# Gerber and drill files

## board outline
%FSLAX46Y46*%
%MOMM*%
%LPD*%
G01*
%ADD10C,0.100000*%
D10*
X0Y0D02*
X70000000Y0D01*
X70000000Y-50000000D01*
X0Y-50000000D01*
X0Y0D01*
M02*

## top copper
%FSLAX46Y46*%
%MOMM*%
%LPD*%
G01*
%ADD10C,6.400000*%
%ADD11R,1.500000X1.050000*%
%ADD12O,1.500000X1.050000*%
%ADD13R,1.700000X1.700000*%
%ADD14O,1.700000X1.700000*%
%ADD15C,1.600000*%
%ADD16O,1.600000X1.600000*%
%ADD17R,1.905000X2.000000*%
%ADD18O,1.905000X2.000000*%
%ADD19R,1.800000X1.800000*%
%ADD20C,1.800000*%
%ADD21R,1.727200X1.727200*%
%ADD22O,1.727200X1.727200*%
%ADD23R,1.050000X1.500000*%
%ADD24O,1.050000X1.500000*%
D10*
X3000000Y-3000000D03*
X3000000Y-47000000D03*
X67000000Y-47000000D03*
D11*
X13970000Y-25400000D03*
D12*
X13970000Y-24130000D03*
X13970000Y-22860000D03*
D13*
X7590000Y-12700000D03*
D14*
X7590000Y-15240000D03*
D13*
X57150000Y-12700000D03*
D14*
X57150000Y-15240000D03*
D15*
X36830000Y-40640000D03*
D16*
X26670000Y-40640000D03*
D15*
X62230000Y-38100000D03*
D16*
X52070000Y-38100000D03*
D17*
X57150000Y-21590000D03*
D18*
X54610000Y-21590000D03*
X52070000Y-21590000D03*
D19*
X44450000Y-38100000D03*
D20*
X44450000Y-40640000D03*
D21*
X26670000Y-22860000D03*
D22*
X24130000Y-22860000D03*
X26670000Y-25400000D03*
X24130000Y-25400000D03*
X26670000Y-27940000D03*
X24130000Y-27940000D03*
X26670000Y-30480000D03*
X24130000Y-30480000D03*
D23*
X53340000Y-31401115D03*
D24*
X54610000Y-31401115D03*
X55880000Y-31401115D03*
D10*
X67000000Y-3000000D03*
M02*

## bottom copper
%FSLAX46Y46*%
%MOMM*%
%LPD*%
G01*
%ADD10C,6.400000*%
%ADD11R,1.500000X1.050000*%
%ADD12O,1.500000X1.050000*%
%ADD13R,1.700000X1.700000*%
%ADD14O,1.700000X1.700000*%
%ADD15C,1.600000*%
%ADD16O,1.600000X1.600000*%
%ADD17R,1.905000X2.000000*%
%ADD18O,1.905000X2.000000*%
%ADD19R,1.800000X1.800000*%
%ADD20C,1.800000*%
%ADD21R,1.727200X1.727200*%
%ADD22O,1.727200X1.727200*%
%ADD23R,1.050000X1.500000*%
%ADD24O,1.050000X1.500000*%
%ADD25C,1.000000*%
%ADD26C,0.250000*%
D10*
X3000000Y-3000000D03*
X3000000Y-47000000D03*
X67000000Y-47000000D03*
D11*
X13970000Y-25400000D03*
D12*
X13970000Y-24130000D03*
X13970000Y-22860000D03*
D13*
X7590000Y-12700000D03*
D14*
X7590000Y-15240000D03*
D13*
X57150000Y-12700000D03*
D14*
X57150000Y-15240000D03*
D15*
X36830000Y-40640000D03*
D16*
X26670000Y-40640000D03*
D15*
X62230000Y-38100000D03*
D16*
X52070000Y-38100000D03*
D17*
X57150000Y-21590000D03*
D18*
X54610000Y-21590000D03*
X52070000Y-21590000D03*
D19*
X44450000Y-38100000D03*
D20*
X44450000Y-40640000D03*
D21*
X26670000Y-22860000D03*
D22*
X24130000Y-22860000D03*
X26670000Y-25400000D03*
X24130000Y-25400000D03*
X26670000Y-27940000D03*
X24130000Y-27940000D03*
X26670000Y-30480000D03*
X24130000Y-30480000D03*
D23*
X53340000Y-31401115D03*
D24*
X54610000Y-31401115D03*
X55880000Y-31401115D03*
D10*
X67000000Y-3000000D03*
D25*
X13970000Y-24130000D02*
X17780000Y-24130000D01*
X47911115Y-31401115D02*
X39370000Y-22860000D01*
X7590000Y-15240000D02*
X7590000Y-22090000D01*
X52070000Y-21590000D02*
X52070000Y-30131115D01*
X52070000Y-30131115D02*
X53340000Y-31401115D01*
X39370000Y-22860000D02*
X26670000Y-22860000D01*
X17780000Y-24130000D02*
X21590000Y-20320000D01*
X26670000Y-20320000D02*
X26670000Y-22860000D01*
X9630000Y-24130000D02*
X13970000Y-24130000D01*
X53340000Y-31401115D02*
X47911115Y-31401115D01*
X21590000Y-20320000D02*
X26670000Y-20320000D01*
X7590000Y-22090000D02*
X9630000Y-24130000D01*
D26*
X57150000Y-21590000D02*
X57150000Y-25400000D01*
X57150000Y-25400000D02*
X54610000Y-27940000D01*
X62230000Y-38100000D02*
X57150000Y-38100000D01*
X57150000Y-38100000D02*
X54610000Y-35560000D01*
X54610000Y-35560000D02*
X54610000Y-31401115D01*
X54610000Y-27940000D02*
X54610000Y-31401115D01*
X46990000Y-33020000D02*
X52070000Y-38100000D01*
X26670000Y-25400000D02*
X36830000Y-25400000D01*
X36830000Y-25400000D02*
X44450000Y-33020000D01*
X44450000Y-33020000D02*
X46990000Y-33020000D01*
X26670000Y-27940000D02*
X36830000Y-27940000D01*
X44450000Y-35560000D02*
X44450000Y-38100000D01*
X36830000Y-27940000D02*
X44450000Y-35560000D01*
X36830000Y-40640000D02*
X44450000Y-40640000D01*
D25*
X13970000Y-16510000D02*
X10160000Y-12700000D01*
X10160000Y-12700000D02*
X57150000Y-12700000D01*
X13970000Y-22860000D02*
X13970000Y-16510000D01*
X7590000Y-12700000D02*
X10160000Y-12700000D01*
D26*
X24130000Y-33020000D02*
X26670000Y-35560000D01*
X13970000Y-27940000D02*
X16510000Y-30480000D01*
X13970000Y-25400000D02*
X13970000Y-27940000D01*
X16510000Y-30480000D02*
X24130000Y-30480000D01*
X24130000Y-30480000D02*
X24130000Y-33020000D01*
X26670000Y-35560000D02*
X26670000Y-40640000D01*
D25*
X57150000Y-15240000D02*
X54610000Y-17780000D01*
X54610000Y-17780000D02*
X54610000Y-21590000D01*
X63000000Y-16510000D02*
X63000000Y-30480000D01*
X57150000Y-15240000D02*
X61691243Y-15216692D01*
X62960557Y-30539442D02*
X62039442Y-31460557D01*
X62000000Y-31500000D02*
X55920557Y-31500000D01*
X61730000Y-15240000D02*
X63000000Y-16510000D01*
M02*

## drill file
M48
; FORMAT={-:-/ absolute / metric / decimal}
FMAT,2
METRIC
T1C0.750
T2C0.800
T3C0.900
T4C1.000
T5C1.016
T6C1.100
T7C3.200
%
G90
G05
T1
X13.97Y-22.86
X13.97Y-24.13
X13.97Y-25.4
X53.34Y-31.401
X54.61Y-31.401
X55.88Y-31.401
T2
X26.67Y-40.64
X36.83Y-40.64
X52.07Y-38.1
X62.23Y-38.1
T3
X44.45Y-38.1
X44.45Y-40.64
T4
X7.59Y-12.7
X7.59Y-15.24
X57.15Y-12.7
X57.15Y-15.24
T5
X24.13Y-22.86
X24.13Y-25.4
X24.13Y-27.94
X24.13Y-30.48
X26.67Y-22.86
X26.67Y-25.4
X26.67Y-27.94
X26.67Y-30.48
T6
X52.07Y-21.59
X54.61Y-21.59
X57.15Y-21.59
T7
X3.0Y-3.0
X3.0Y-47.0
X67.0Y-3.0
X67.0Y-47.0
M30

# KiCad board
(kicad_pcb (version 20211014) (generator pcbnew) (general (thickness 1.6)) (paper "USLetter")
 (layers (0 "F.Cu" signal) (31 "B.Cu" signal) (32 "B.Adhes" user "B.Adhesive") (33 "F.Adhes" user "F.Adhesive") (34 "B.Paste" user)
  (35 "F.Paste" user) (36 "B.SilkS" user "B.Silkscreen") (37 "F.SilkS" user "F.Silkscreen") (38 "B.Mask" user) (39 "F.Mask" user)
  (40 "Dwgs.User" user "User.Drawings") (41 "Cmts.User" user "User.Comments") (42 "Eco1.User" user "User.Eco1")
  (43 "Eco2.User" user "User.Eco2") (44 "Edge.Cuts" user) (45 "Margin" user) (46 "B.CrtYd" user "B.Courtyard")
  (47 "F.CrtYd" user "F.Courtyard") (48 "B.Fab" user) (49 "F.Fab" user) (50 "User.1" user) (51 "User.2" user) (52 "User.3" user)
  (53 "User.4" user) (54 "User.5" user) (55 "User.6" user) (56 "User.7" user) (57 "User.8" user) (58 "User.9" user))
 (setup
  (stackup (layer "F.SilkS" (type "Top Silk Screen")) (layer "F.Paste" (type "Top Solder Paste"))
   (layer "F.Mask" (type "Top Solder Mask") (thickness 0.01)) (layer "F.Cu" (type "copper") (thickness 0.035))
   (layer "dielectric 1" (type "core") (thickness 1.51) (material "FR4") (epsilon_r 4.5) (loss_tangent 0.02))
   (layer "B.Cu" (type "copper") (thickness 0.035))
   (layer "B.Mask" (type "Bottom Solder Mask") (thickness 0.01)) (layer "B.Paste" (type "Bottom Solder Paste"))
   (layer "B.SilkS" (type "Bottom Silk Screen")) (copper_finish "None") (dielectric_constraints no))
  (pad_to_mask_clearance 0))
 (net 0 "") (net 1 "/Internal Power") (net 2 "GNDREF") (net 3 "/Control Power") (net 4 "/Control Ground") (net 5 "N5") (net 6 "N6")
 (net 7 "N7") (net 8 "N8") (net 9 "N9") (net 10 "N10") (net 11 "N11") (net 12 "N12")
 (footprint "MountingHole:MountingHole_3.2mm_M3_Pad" (layer "F.Cu") (at 3 3)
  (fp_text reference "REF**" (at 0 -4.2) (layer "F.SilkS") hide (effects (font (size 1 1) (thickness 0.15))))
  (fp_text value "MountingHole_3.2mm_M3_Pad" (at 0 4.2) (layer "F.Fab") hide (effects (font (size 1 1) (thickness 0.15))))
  (pad "1" thru_hole circle (at 0 0) (size 6.4 6.4) (drill 3.2) (layers *.Cu *.Mask)))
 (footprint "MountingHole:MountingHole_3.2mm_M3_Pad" (layer "F.Cu") (at 3 47)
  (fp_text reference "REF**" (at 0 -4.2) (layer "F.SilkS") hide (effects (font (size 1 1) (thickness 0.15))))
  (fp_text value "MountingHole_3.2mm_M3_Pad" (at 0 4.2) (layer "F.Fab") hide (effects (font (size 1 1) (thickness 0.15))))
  (pad "1" thru_hole circle (at 0 0) (size 6.4 6.4) (drill 3.2) (layers *.Cu *.Mask)))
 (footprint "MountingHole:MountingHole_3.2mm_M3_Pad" (layer "F.Cu") (at 67 47)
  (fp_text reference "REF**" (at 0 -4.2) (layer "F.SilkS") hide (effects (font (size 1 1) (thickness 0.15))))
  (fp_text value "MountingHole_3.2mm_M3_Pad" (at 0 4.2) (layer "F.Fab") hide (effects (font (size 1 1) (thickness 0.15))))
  (pad "1" thru_hole circle (at 0 0) (size 6.4 6.4) (drill 3.2) (layers *.Cu *.Mask)))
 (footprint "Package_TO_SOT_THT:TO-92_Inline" (layer "F.Cu") (at 13.97 25.4 90)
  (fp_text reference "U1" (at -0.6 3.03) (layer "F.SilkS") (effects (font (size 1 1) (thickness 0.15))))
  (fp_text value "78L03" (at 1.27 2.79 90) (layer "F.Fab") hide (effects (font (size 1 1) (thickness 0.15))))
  (pad "1" thru_hole rect (at 0 0 90) (size 1.05 1.5) (drill 0.75) (layers *.Cu *.Mask) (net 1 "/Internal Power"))
  (pad "2" thru_hole oval (at 1.27 0 90) (size 1.05 1.5) (drill 0.75) (layers *.Cu *.Mask) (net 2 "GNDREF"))
  (pad "3" thru_hole oval (at 2.54 0 90) (size 1.05 1.5) (drill 0.75) (layers *.Cu *.Mask) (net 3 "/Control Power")))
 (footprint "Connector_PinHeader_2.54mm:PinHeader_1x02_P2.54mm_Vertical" (layer "F.Cu") (at 7.59 12.7)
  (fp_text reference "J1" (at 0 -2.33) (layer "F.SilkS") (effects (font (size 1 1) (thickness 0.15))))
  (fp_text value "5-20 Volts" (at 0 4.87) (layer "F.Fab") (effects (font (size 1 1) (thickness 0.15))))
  (pad "1" thru_hole rect (at 0 0) (size 1.7 1.7) (drill 1) (layers *.Cu *.Mask) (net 3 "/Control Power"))
  (pad "2" thru_hole oval (at 0 2.54) (size 1.7 1.7) (drill 1) (layers *.Cu *.Mask) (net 2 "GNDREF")))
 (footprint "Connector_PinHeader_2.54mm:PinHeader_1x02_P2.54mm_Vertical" (layer "F.Cu") (at 57.15 12.7)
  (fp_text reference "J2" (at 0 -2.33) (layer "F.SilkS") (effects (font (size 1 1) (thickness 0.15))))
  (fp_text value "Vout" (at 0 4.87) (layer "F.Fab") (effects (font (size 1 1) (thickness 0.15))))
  (pad "1" thru_hole rect (at 0 0) (size 1.7 1.7) (drill 1) (layers *.Cu *.Mask) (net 3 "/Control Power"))
  (pad "2" thru_hole oval (at 0 2.54) (size 1.7 1.7) (drill 1) (layers *.Cu *.Mask) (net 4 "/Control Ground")))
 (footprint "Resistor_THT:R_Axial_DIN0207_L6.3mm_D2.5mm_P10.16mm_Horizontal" (layer "F.Cu") (at 36.83 40.64 180)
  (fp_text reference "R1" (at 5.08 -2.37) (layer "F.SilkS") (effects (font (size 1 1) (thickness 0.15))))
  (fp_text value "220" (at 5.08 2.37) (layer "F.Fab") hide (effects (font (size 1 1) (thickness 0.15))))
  (pad "1" thru_hole circle (at 0 0 180) (size 1.6 1.6) (drill 0.8) (layers *.Cu *.Mask) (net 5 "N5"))
  (pad "2" thru_hole oval (at 10.16 0 180) (size 1.6 1.6) (drill 0.8) (layers *.Cu *.Mask) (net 1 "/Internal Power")))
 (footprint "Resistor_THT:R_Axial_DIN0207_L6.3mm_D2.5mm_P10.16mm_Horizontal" (layer "F.Cu") (at 62.23 38.1 180)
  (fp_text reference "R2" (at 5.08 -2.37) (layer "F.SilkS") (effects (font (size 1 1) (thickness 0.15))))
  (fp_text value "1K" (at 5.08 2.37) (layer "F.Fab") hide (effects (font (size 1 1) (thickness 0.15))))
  (pad "1" thru_hole circle (at 0 0 180) (size 1.6 1.6) (drill 0.8) (layers *.Cu *.Mask) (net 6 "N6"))
  (pad "2" thru_hole oval (at 10.16 0 180) (size 1.6 1.6) (drill 0.8) (layers *.Cu *.Mask) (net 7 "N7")))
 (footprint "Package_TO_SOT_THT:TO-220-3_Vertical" (layer "F.Cu") (at 57.15 21.59 180)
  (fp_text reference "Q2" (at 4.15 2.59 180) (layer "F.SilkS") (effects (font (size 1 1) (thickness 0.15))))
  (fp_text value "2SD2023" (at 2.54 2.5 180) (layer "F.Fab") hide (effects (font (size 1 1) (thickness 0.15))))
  (pad "1" thru_hole rect (at 0 0 180) (size 1.905 2) (drill 1.1) (layers *.Cu *.Mask) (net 6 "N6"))
  (pad "2" thru_hole oval (at 2.54 0 180) (size 1.905 2) (drill 1.1) (layers *.Cu *.Mask) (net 4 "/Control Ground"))
  (pad "3" thru_hole oval (at 5.08 0 180) (size 1.905 2) (drill 1.1) (layers *.Cu *.Mask) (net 2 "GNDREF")))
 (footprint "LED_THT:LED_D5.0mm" (layer "F.Cu") (at 44.45 38.1 -90)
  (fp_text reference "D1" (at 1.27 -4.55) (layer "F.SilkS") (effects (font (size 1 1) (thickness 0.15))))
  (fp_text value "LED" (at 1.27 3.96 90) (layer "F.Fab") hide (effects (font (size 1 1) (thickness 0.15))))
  (pad "1" thru_hole rect (at 0 0 270) (size 1.8 1.8) (drill 0.9) (layers *.Cu *.Mask) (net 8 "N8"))
  (pad "2" thru_hole circle (at 2.54 0 270) (size 1.8 1.8) (drill 0.9) (layers *.Cu *.Mask) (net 5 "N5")))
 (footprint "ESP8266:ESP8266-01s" (layer "F.Cu") (at 24.13 22.86)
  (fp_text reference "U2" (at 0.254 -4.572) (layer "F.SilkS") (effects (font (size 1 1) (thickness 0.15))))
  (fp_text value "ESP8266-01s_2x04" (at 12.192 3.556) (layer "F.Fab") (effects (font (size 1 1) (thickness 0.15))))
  (pad "1" thru_hole rect (at 2.54 0) (size 1.7272 1.7272) (drill 1.016) (layers *.Cu *.Mask) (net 2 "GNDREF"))
  (pad "2" thru_hole oval (at 0 0) (size 1.7272 1.7272) (drill 1.016) (layers *.Cu *.Mask) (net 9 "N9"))
  (pad "3" thru_hole oval (at 2.54 2.54) (size 1.7272 1.7272) (drill 1.016) (layers *.Cu *.Mask) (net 7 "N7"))
  (pad "4" thru_hole oval (at 0 2.54) (size 1.7272 1.7272) (drill 1.016) (layers *.Cu *.Mask) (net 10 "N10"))
  (pad "5" thru_hole oval (at 2.54 5.08) (size 1.7272 1.7272) (drill 1.016) (layers *.Cu *.Mask) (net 8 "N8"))
  (pad "6" thru_hole oval (at 0 5.08) (size 1.7272 1.7272) (drill 1.016) (layers *.Cu *.Mask) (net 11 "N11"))
  (pad "7" thru_hole oval (at 2.54 7.62) (size 1.7272 1.7272) (drill 1.016) (layers *.Cu *.Mask) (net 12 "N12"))
  (pad "8" thru_hole oval (at 0 7.62) (size 1.7272 1.7272) (drill 1.016) (layers *.Cu *.Mask) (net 1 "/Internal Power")))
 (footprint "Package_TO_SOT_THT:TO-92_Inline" (layer "F.Cu") (at 53.34 31.401115)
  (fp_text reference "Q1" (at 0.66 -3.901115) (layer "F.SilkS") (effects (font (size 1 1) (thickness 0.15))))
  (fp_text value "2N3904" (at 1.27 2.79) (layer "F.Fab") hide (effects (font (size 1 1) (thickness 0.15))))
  (pad "1" thru_hole rect (at 0 0) (size 1.05 1.5) (drill 0.75) (layers *.Cu *.Mask) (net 2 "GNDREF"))
  (pad "2" thru_hole oval (at 1.27 0) (size 1.05 1.5) (drill 0.75) (layers *.Cu *.Mask) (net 6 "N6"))
  (pad "3" thru_hole oval (at 2.54 0) (size 1.05 1.5) (drill 0.75) (layers *.Cu *.Mask) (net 4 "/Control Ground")))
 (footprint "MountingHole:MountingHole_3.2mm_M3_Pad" (layer "F.Cu") (at 67 3)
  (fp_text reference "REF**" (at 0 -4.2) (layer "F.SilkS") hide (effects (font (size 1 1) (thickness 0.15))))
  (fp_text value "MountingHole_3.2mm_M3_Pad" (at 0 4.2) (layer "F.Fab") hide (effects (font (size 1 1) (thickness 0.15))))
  (pad "1" thru_hole circle (at 0 0) (size 6.4 6.4) (drill 3.2) (layers *.Cu *.Mask)))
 (gr_rect (start 0 0) (end 70 50) (layer "Edge.Cuts") (width 0.1) (fill none))
 (segment (start 13.97 24.13) (end 17.78 24.13) (width 1) (layer "B.Cu") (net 2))
 (segment (start 47.911115 31.401115) (end 39.37 22.86) (width 1) (layer "B.Cu") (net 2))
 (segment (start 7.59 15.24) (end 7.59 22.09) (width 1) (layer "B.Cu") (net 2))
 (segment (start 52.07 21.59) (end 52.07 30.131115) (width 1) (layer "B.Cu") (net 2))
 (segment (start 52.07 30.131115) (end 53.34 31.401115) (width 1) (layer "B.Cu") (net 2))
 (segment (start 39.37 22.86) (end 26.67 22.86) (width 1) (layer "B.Cu") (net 2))
 (segment (start 17.78 24.13) (end 21.59 20.32) (width 1) (layer "B.Cu") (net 2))
 (segment (start 26.67 20.32) (end 26.67 22.86) (width 1) (layer "B.Cu") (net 2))
 (segment (start 9.63 24.13) (end 13.97 24.13) (width 1) (layer "B.Cu") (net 2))
 (segment (start 53.34 31.401115) (end 47.911115 31.401115) (width 1) (layer "B.Cu") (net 2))
 (segment (start 21.59 20.32) (end 26.67 20.32) (width 1) (layer "B.Cu") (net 2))
 (segment (start 7.59 22.09) (end 9.63 24.13) (width 1) (layer "B.Cu") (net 2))
 (segment (start 57.15 21.59) (end 57.15 25.4) (width 0.25) (layer "B.Cu") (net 6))
 (segment (start 57.15 25.4) (end 54.61 27.94) (width 0.25) (layer "B.Cu") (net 6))
 (segment (start 62.23 38.1) (end 57.15 38.1) (width 0.25) (layer "B.Cu") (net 6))
 (segment (start 57.15 38.1) (end 54.61 35.56) (width 0.25) (layer "B.Cu") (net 6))
 (segment (start 54.61 35.56) (end 54.61 31.401115) (width 0.25) (layer "B.Cu") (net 6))
 (segment (start 54.61 27.94) (end 54.61 31.401115) (width 0.25) (layer "B.Cu") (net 6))
 (segment (start 46.99 33.02) (end 52.07 38.1) (width 0.25) (layer "B.Cu") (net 7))
 (segment (start 26.67 25.4) (end 36.83 25.4) (width 0.25) (layer "B.Cu") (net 7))
 (segment (start 36.83 25.4) (end 44.45 33.02) (width 0.25) (layer "B.Cu") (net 7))
 (segment (start 44.45 33.02) (end 46.99 33.02) (width 0.25) (layer "B.Cu") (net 7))
 (segment (start 26.67 27.94) (end 36.83 27.94) (width 0.25) (layer "B.Cu") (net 8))
 (segment (start 44.45 35.56) (end 44.45 38.1) (width 0.25) (layer "B.Cu") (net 8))
 (segment (start 36.83 27.94) (end 44.45 35.56) (width 0.25) (layer "B.Cu") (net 8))
 (segment (start 36.83 40.64) (end 44.45 40.64) (width 0.25) (layer "B.Cu") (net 5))
 (segment (start 13.97 16.51) (end 10.16 12.7) (width 1) (layer "B.Cu") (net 3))
 (segment (start 10.16 12.7) (end 57.15 12.7) (width 1) (layer "B.Cu") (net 3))
 (segment (start 13.97 22.86) (end 13.97 16.51) (width 1) (layer "B.Cu") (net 3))
 (segment (start 7.59 12.7) (end 10.16 12.7) (width 1) (layer "B.Cu") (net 3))
 (segment (start 24.13 33.02) (end 26.67 35.56) (width 0.25) (layer "B.Cu") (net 1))
 (segment (start 13.97 27.94) (end 16.51 30.48) (width 0.25) (layer "B.Cu") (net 1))
 (segment (start 13.97 25.4) (end 13.97 27.94) (width 0.25) (layer "B.Cu") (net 1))
 (segment (start 16.51 30.48) (end 24.13 30.48) (width 0.25) (layer "B.Cu") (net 1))
 (segment (start 24.13 30.48) (end 24.13 33.02) (width 0.25) (layer "B.Cu") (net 1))
 (segment (start 26.67 35.56) (end 26.67 40.64) (width 0.25) (layer "B.Cu") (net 1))
 (segment (start 57.15 15.24) (end 54.61 17.78) (width 1) (layer "B.Cu") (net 4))
 (segment (start 54.61 17.78) (end 54.61 21.59) (width 1) (layer "B.Cu") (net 4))
 (segment (start 63 16.51) (end 63 30.48) (width 1) (layer "B.Cu") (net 4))
 (segment (start 57.15 15.24) (end 61.691243 15.216692) (width 1) (layer "B.Cu") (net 4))
 (segment (start 62.960557 30.539442) (end 62.039442 31.460557) (width 1) (layer "B.Cu") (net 4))
 (segment (start 62 31.5) (end 55.920557 31.5) (width 1) (layer "B.Cu") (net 4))
 (segment (start 61.73 15.24) (end 63 16.51) (width 1) (layer "B.Cu") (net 4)))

